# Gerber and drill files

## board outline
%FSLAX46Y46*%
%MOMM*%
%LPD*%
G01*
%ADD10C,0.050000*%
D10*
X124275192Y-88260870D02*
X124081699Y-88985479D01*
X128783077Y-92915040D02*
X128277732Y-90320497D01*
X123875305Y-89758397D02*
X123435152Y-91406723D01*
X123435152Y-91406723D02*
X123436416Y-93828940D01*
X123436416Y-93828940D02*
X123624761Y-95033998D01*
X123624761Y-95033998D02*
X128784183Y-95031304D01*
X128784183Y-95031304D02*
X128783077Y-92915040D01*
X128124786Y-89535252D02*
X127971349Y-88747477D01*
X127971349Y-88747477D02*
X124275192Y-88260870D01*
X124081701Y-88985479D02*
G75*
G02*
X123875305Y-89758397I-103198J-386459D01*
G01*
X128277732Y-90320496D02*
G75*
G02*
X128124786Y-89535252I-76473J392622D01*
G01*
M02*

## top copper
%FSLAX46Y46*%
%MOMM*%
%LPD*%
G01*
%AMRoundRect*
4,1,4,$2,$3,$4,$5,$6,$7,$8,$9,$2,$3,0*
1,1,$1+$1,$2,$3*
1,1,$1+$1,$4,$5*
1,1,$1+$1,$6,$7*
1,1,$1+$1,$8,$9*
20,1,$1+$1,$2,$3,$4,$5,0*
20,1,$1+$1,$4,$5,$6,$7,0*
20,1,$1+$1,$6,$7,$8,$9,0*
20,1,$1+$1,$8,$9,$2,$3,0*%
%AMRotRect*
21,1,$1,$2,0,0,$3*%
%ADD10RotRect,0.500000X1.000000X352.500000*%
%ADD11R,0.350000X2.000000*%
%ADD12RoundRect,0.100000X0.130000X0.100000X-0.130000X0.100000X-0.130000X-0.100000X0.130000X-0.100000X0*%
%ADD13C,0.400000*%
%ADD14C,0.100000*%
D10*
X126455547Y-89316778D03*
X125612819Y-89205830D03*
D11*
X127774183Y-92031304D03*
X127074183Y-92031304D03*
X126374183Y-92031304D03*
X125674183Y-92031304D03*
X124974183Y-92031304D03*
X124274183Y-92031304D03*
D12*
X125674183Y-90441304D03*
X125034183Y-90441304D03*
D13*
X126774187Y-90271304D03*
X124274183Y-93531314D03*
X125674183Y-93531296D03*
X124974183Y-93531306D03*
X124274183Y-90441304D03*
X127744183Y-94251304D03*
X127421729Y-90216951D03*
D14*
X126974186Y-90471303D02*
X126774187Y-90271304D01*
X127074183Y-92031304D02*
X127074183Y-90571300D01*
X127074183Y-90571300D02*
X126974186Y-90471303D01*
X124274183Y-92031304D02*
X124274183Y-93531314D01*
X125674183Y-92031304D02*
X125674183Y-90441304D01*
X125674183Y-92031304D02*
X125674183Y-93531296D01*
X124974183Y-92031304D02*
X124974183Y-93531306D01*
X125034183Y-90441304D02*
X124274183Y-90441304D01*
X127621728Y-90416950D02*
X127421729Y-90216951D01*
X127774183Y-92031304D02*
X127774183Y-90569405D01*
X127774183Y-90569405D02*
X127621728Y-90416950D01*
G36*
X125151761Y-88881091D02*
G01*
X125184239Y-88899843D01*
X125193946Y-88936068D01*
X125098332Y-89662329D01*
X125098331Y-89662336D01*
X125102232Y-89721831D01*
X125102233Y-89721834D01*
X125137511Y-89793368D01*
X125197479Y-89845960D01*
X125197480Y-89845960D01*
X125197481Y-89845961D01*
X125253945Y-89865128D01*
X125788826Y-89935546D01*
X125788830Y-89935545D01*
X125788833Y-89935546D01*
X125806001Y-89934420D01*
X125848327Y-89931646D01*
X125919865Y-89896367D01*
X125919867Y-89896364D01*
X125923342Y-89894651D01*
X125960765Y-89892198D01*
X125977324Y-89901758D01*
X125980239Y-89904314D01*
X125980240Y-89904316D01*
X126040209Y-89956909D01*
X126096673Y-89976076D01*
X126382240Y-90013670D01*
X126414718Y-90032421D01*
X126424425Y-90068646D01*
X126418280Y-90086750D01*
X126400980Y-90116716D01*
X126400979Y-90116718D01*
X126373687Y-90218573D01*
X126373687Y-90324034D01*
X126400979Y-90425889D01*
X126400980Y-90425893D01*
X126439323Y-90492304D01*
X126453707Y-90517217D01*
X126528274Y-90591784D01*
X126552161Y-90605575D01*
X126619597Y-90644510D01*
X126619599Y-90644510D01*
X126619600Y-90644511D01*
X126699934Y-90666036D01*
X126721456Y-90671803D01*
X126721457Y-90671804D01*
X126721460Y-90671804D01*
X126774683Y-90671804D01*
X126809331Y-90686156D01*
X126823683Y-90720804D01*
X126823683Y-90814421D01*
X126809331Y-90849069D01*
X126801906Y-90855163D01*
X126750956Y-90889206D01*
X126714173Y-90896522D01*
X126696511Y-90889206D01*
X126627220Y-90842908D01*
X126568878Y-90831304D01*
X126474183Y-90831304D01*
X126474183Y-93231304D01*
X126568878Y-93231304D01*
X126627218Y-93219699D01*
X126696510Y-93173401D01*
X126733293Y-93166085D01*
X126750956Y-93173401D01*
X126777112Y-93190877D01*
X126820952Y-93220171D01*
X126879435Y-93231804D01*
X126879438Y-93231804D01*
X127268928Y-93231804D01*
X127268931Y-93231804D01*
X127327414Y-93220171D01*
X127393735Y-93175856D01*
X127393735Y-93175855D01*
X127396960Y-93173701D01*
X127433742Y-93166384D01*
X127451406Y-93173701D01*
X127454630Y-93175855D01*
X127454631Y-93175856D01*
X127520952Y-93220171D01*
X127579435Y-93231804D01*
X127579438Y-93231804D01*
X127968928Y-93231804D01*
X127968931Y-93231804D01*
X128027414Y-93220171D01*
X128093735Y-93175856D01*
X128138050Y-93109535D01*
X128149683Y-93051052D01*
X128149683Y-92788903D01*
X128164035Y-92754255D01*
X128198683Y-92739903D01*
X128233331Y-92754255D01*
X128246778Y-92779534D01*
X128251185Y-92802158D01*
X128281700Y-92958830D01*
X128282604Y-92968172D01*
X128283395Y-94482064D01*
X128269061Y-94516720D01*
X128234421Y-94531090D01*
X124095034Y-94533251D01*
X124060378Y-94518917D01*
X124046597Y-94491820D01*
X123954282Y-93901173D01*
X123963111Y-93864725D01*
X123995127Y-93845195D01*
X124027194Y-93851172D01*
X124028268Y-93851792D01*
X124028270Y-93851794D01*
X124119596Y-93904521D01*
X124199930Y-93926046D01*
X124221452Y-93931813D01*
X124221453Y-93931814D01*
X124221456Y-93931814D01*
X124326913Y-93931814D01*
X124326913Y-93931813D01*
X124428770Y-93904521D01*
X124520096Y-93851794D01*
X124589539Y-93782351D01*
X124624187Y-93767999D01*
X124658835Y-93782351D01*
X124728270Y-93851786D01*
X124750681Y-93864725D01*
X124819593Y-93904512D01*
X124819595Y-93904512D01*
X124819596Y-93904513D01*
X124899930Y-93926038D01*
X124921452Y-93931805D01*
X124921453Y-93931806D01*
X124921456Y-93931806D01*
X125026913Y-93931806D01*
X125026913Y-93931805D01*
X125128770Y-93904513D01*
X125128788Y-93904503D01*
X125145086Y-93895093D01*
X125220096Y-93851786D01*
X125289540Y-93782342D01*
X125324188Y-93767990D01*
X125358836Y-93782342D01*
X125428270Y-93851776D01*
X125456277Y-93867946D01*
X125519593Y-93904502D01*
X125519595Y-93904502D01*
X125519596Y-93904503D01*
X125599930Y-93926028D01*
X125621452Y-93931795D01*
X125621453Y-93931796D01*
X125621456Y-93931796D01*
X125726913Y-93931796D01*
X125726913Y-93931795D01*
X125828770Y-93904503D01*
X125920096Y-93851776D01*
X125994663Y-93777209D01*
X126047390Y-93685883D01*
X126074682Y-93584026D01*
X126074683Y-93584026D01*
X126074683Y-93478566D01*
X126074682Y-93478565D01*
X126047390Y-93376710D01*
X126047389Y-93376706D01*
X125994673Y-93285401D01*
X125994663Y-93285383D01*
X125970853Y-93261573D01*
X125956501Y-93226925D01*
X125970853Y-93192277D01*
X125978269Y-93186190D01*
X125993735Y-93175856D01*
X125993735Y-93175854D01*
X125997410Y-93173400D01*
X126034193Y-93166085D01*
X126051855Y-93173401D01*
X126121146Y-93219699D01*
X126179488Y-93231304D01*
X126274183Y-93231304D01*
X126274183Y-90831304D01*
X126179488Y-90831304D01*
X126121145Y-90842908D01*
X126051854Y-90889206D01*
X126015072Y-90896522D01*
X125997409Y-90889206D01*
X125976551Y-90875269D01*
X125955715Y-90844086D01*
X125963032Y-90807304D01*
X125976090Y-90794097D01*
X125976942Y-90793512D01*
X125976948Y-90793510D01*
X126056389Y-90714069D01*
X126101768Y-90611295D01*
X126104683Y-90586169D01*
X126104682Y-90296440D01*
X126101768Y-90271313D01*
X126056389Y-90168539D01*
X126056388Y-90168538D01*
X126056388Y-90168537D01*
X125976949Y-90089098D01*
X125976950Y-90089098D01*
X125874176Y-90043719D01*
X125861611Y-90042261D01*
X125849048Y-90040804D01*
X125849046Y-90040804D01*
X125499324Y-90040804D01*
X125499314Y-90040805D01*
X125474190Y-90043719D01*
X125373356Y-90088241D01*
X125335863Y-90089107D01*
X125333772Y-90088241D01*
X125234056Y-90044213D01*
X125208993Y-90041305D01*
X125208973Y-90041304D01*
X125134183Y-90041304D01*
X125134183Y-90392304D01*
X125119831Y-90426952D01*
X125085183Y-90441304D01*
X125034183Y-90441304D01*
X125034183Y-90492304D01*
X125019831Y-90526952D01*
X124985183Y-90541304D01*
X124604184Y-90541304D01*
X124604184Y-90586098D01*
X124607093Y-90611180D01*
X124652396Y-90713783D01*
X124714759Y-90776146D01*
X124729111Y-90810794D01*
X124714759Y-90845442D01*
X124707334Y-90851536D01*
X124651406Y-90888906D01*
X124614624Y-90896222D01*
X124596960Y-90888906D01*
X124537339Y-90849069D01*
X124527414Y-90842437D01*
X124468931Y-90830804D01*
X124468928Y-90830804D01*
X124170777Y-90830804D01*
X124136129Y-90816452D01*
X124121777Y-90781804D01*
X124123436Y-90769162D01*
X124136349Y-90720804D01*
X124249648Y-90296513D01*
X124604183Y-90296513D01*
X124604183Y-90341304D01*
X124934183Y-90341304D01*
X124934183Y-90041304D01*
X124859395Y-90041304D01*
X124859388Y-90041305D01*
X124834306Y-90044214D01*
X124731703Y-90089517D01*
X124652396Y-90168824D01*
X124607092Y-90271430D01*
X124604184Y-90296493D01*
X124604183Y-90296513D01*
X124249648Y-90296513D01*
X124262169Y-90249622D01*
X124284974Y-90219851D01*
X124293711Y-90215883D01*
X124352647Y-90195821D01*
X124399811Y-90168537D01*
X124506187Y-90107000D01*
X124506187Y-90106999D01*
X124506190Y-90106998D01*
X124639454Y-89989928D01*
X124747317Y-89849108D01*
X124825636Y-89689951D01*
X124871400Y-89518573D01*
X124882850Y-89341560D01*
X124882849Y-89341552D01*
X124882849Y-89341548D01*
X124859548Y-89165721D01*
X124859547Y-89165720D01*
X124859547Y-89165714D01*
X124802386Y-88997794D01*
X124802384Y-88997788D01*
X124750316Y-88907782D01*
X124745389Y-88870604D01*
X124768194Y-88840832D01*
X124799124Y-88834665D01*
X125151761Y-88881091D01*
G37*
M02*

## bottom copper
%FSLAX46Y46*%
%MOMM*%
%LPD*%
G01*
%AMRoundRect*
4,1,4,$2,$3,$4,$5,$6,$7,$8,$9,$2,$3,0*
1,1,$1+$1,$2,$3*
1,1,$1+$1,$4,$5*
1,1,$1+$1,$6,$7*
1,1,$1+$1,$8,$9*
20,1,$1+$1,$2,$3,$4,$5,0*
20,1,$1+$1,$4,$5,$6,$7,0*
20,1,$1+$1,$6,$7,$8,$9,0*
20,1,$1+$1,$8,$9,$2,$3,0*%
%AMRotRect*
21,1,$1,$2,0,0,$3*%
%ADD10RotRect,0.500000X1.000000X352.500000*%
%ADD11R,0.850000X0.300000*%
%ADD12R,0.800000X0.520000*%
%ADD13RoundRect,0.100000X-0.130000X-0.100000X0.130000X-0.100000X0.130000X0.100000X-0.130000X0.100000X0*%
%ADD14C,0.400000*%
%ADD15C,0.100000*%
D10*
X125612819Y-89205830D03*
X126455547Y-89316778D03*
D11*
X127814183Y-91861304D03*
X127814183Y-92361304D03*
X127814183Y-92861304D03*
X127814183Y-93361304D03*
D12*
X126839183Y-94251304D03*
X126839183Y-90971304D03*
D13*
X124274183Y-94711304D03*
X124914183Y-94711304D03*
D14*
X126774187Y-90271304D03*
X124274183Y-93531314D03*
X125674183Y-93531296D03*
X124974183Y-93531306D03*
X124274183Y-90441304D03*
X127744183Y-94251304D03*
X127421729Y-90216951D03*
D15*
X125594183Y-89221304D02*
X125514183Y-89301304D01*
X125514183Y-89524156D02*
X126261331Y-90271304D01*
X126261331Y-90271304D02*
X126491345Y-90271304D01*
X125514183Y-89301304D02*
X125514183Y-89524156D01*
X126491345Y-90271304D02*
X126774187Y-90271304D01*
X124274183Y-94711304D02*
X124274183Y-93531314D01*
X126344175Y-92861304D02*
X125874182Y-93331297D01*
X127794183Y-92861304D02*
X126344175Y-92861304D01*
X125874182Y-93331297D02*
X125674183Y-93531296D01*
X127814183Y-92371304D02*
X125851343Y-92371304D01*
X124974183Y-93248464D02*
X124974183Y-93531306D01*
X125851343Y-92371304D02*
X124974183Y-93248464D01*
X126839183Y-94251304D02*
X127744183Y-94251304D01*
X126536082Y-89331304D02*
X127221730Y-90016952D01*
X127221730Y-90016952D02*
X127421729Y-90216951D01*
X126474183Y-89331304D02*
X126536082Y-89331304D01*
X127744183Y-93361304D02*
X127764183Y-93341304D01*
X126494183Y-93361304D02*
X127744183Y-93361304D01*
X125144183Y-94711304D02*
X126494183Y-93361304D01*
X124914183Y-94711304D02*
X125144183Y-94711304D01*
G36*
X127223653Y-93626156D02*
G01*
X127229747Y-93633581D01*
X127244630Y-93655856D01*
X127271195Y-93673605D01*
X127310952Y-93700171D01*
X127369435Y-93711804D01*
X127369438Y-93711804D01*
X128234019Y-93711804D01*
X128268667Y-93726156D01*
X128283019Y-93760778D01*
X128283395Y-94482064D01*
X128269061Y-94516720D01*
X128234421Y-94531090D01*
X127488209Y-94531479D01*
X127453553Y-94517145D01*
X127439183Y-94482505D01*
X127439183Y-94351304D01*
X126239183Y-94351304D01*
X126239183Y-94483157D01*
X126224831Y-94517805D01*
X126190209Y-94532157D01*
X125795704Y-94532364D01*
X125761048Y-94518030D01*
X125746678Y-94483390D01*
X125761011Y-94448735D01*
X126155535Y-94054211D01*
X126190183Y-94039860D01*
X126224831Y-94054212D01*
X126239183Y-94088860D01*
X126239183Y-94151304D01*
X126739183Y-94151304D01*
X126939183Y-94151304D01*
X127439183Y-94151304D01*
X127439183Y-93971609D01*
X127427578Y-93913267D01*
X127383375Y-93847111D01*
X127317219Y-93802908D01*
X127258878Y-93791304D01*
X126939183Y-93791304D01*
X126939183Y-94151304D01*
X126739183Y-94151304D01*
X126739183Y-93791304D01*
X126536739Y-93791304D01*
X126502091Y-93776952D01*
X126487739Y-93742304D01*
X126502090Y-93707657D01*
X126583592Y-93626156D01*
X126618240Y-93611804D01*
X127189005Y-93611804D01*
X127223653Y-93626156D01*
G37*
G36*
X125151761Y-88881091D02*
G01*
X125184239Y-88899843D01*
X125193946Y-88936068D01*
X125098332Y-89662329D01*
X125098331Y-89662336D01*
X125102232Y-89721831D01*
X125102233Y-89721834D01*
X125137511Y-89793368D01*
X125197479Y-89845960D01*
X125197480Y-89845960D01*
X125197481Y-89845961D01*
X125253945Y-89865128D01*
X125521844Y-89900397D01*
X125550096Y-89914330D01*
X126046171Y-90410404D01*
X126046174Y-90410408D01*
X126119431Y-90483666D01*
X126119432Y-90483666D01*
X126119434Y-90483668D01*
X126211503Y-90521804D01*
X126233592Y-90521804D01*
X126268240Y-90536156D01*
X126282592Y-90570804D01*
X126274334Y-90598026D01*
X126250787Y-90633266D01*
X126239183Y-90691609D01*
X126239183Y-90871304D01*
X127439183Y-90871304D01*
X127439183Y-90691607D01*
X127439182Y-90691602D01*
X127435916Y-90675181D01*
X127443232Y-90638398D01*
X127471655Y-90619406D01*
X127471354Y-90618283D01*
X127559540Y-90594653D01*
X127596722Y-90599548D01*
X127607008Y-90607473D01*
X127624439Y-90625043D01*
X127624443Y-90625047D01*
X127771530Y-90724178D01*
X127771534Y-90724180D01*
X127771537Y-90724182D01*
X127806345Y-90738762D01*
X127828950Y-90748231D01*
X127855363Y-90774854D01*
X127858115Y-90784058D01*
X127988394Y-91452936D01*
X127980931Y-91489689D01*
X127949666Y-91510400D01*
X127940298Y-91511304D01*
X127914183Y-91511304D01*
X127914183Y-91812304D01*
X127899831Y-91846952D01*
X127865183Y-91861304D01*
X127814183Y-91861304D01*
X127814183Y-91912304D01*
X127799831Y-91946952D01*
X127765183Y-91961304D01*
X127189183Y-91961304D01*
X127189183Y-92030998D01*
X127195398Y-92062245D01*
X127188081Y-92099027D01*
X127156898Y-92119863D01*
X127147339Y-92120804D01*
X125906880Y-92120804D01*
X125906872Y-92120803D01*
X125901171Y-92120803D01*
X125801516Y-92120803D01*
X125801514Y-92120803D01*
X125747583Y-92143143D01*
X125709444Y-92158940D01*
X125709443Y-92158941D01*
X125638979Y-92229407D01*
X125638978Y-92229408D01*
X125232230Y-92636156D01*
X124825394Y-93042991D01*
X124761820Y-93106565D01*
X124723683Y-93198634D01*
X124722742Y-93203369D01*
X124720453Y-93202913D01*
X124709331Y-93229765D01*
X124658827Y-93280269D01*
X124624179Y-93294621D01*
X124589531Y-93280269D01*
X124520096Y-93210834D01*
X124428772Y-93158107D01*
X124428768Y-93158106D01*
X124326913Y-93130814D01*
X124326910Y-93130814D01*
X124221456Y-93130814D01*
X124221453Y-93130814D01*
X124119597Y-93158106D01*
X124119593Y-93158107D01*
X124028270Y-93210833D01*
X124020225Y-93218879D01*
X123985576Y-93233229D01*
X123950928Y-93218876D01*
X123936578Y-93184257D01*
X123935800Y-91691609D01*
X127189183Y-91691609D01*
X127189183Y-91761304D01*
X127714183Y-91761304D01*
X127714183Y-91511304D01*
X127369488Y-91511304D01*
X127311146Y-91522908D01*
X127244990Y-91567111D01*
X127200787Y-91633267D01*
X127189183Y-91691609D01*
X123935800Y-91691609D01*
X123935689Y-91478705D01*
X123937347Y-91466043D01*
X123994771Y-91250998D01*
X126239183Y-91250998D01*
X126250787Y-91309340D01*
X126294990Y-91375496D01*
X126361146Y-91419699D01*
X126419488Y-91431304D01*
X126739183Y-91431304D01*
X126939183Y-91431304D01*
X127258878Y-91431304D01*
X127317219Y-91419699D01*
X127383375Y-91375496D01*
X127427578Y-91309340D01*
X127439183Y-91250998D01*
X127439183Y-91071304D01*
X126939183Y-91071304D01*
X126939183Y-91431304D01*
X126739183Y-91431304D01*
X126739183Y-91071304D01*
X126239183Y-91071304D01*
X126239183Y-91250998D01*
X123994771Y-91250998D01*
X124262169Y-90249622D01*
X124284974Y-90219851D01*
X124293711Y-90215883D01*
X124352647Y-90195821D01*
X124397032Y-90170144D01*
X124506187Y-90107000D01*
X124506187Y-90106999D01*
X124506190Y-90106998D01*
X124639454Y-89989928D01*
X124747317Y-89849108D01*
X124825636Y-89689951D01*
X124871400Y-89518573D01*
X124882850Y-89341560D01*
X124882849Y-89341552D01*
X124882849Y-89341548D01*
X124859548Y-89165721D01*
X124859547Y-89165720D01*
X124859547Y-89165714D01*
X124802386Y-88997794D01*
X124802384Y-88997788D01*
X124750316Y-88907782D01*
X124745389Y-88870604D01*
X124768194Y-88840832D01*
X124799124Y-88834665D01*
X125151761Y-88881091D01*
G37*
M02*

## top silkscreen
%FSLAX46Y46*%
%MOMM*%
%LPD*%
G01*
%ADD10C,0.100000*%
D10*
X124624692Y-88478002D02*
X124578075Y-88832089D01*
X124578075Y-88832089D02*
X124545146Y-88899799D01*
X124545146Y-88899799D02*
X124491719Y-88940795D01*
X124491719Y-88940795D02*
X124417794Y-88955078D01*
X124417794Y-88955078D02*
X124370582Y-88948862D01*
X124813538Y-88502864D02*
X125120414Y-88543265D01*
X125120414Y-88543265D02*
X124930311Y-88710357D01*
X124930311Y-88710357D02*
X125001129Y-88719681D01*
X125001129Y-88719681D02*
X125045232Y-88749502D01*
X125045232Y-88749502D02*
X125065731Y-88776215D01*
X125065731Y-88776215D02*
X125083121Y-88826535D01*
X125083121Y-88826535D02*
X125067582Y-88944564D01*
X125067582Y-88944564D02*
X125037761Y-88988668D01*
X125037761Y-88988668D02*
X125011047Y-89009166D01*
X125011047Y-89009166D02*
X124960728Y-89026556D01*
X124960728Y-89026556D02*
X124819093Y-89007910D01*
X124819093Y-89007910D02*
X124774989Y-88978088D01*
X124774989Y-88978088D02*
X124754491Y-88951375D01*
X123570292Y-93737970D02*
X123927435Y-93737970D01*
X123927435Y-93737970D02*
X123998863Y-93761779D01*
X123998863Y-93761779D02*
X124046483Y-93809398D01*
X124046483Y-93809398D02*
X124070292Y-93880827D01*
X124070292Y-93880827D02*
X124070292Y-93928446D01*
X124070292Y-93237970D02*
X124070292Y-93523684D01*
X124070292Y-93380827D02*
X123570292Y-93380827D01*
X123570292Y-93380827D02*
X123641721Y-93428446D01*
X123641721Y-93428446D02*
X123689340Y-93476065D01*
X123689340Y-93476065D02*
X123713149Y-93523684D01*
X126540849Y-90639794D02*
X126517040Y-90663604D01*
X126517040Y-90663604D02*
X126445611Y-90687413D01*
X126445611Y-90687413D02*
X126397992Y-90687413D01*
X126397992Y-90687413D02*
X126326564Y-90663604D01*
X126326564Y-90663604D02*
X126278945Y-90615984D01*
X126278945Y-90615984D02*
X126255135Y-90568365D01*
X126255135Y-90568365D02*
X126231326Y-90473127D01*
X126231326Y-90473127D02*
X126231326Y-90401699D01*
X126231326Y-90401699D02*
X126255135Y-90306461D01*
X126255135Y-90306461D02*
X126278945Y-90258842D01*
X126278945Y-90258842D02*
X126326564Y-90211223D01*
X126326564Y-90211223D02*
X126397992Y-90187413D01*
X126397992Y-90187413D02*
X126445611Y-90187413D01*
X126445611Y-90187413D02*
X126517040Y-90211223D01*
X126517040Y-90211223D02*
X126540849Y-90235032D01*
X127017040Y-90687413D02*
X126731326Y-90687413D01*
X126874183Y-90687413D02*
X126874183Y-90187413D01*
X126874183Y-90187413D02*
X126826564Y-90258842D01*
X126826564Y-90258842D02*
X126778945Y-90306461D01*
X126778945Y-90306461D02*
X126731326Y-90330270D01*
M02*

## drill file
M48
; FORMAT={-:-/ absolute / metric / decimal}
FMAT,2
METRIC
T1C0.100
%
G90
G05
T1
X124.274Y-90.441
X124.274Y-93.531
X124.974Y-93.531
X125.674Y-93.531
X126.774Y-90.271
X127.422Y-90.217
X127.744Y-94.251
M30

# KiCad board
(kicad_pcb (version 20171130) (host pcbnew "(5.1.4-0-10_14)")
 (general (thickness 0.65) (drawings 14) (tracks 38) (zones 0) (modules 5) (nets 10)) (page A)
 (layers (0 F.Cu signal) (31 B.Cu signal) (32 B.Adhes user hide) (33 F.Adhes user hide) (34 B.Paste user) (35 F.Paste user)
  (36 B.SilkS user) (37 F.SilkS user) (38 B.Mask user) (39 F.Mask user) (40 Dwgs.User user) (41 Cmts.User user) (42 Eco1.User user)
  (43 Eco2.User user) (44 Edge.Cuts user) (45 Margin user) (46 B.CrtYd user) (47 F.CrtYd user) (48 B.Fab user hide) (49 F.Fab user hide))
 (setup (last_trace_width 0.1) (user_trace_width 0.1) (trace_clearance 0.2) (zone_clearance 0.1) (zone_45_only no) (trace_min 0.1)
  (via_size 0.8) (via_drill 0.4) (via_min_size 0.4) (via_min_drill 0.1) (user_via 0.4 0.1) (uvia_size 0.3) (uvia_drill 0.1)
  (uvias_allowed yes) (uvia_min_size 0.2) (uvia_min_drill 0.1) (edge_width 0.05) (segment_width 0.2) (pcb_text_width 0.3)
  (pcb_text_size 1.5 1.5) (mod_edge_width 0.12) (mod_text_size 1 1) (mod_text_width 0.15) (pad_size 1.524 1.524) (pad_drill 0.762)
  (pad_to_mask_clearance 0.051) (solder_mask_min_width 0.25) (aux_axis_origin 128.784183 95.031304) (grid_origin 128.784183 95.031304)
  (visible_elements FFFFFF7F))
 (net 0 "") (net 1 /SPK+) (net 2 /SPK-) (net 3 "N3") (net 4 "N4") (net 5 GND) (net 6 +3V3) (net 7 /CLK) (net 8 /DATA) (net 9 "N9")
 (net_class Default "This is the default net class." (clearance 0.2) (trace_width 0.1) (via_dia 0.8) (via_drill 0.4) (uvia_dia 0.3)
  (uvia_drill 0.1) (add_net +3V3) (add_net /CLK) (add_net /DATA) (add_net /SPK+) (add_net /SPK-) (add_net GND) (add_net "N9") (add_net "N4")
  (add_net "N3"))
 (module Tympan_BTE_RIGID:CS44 (layer F.Cu) (at 126.034183 89.261304 352.5)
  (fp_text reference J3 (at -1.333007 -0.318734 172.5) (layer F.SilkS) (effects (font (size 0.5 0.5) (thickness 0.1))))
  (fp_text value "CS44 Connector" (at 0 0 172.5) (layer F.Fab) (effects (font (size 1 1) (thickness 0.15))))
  (pad 4 smd rect (at -0.425 0 352.5) (size 0.5 1) (layers B.Cu B.Mask) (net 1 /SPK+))
  (pad 3 smd rect (at 0.425 0 352.5) (size 0.5 1) (layers B.Cu B.Mask) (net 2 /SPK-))
  (pad 2 smd rect (at 0.425 0 352.5) (size 0.5 1) (layers F.Cu F.Mask) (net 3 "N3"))
  (pad 1 smd rect (at -0.425 0 352.5) (size 0.5 1) (layers F.Cu F.Mask) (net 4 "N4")))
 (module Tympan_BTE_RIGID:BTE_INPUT (layer F.Cu) (at 126.024183 92.031304 90)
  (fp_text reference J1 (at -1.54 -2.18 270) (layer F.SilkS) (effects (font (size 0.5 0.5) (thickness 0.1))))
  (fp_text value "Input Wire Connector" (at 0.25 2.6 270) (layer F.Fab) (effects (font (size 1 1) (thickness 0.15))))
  (pad 6 smd rect (at 0 1.75 90) (size 2 0.35) (layers F.Cu F.Mask) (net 2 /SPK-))
  (pad 5 smd rect (at 0 1.05 90) (size 2 0.35) (layers F.Cu F.Mask) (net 1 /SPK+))
  (pad 4 smd rect (at 0 0.35 90) (size 2 0.35) (layers F.Cu F.Mask) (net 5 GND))
  (pad 3 smd rect (at 0 -0.35 90) (size 2 0.35) (layers F.Cu F.Mask) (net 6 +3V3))
  (pad 2 smd rect (at 0 -1.05 90) (size 2 0.35) (layers F.Cu F.Mask) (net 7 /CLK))
  (pad 1 smd rect (at 0 -1.75 90) (size 2 0.35) (layers F.Cu F.Mask) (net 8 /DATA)))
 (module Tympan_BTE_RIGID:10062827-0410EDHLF (layer B.Cu) (at 127.814183 92.611304 90)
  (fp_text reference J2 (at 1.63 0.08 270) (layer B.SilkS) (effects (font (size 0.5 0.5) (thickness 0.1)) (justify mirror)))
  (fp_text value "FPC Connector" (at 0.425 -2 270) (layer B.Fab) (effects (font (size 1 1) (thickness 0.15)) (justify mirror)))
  (pad 1 smd rect (at 0.75 0 90) (size 0.3 0.85) (layers B.Cu B.Paste B.Mask) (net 5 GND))
  (pad 2 smd rect (at 0.25 0 90) (size 0.3 0.85) (layers B.Cu B.Paste B.Mask) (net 7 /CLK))
  (pad 3 smd rect (at -0.25 0 90) (size 0.3 0.85) (layers B.Cu B.Paste B.Mask) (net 6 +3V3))
  (pad 4 smd rect (at -0.75 0 90) (size 0.3 0.85) (layers B.Cu B.Paste B.Mask) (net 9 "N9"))
  (pad 5 smd rect (at -1.64 -0.975 90) (size 0.52 0.8) (layers B.Cu B.Paste B.Mask) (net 5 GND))
  (pad 6 smd rect (at 1.64 -0.975 90) (size 0.52 0.8) (layers B.Cu B.Paste B.Mask) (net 5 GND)))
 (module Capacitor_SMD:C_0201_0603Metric (layer F.Cu) (at 125.354183 90.441304 180)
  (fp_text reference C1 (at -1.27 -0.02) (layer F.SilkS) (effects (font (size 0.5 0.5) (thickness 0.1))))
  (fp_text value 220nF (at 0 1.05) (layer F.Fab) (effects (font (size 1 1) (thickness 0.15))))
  (pad "" smd roundrect (at -0.345 0 180) (size 0.318 0.36) (layers F.Paste) (roundrect_rratio 0.25))
  (pad "" smd roundrect (at 0.345 0 180) (size 0.318 0.36) (layers F.Paste) (roundrect_rratio 0.25))
  (pad 1 smd roundrect (at -0.32 0 180) (size 0.46 0.4) (layers F.Cu F.Mask) (roundrect_rratio 0.25) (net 6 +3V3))
  (pad 2 smd roundrect (at 0.32 0 180) (size 0.46 0.4) (layers F.Cu F.Mask) (roundrect_rratio 0.25) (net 5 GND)))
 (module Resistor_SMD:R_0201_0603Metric (layer B.Cu) (at 124.594183 94.711304)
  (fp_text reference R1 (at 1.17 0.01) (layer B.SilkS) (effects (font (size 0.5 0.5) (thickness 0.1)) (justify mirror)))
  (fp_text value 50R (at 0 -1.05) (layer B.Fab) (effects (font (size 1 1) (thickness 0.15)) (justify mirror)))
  (pad "" smd roundrect (at -0.345 0) (size 0.318 0.36) (layers B.Paste) (roundrect_rratio 0.25))
  (pad "" smd roundrect (at 0.345 0) (size 0.318 0.36) (layers B.Paste) (roundrect_rratio 0.25))
  (pad 1 smd roundrect (at -0.32 0) (size 0.46 0.4) (layers B.Cu B.Mask) (roundrect_rratio 0.25) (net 8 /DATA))
  (pad 2 smd roundrect (at 0.32 0) (size 0.46 0.4) (layers B.Cu B.Mask) (roundrect_rratio 0.25) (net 9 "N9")))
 (gr_line (start 124.275192 88.26087) (end 124.081699 88.985479) (layer Edge.Cuts) (width 0.05))
 (gr_line (start 128.783077 92.91504) (end 128.277732 90.320497) (layer Edge.Cuts) (width 0.05))
 (gr_line (start 123.875305 89.758397) (end 123.435152 91.406723) (layer Edge.Cuts) (width 0.05))
 (gr_line (start 123.435152 91.406723) (end 123.436416 93.82894) (layer Edge.Cuts) (width 0.05))
 (gr_line (start 123.436416 93.82894) (end 123.624761 95.033998) (layer Edge.Cuts) (width 0.05))
 (gr_line (start 123.624761 95.033998) (end 128.784183 95.031304) (layer Edge.Cuts) (width 0.05))
 (gr_line (start 128.784183 95.031304) (end 128.783077 92.91504) (layer Edge.Cuts) (width 0.05))
 (gr_line (start 128.124786 89.535252) (end 127.971349 88.747477) (layer Edge.Cuts) (width 0.05))
 (gr_line (start 127.971349 88.747477) (end 124.275192 88.26087) (layer Edge.Cuts) (width 0.05))
 (gr_arc (start 123.978503 89.371938) (end 123.875305 89.758397) (angle -180) (layer Edge.Cuts) (width 0.05))
 (gr_arc (start 128.201259 89.927874) (end 128.124786 89.535252) (angle -180) (layer Edge.Cuts) (width 0.05))
 (via (at 126.774187 90.271304) (size 0.4) (drill 0.1) (layers F.Cu B.Cu) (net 1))
 (segment (start 126.974186 90.471303) (end 126.774187 90.271304) (width 0.1) (layer F.Cu) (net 1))
 (segment (start 125.594183 89.221304) (end 125.514183 89.301304) (width 0.1) (layer B.Cu) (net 1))
 (segment (start 127.074183 92.031304) (end 127.074183 90.5713) (width 0.1) (layer F.Cu) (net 1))
 (segment (start 127.074183 90.5713) (end 126.974186 90.471303) (width 0.1) (layer F.Cu) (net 1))
 (segment (start 125.514183 89.524156) (end 126.261331 90.271304) (width 0.1) (layer B.Cu) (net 1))
 (segment (start 126.261331 90.271304) (end 126.491345 90.271304) (width 0.1) (layer B.Cu) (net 1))
 (segment (start 125.514183 89.301304) (end 125.514183 89.524156) (width 0.1) (layer B.Cu) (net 1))
 (segment (start 126.491345 90.271304) (end 126.774187 90.271304) (width 0.1) (layer B.Cu) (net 1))
 (via (at 124.274183 93.531314) (size 0.4) (drill 0.1) (layers F.Cu B.Cu) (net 8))
 (segment (start 124.274183 92.031304) (end 124.274183 93.531314) (width 0.1) (layer F.Cu) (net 8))
 (segment (start 124.274183 94.711304) (end 124.274183 93.531314) (width 0.1) (layer B.Cu) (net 8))
 (segment (start 125.674183 92.031304) (end 125.674183 90.441304) (width 0.1) (layer F.Cu) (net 6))
 (via (at 125.674183 93.531296) (size 0.4) (drill 0.1) (layers F.Cu B.Cu) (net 6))
 (segment (start 126.344175 92.861304) (end 125.874182 93.331297) (width 0.1) (layer B.Cu) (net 6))
 (segment (start 125.674183 92.031304) (end 125.674183 93.531296) (width 0.1) (layer F.Cu) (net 6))
 (segment (start 127.794183 92.861304) (end 126.344175 92.861304) (width 0.1) (layer B.Cu) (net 6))
 (segment (start 125.874182 93.331297) (end 125.674183 93.531296) (width 0.1) (layer B.Cu) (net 6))
 (via (at 124.974183 93.531306) (size 0.4) (drill 0.1) (layers F.Cu B.Cu) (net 7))
 (segment (start 124.974183 92.031304) (end 124.974183 93.531306) (width 0.1) (layer F.Cu) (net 7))
 (segment (start 127.814183 92.371304) (end 125.851343 92.371304) (width 0.1) (layer B.Cu) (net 7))
 (segment (start 124.974183 93.248464) (end 124.974183 93.531306) (width 0.1) (layer B.Cu) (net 7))
 (segment (start 125.851343 92.371304) (end 124.974183 93.248464) (width 0.1) (layer B.Cu) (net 7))
 (via (at 124.274183 90.441304) (size 0.4) (drill 0.1) (layers F.Cu B.Cu) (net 5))
 (segment (start 125.034183 90.441304) (end 124.274183 90.441304) (width 0.1) (layer F.Cu) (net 5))
 (via (at 127.744183 94.251304) (size 0.4) (drill 0.1) (layers F.Cu B.Cu) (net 5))
 (segment (start 126.839183 94.251304) (end 127.744183 94.251304) (width 0.1) (layer B.Cu) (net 5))
 (segment (start 126.536082 89.331304) (end 127.22173 90.016952) (width 0.1) (layer B.Cu) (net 2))
 (segment (start 127.621728 90.41695) (end 127.421729 90.216951) (width 0.1) (layer F.Cu) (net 2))
 (via (at 127.421729 90.216951) (size 0.4) (drill 0.1) (layers F.Cu B.Cu) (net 2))
 (segment (start 127.22173 90.016952) (end 127.421729 90.216951) (width 0.1) (layer B.Cu) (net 2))
 (segment (start 127.774183 92.031304) (end 127.774183 90.569405) (width 0.1) (layer F.Cu) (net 2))
 (segment (start 127.774183 90.569405) (end 127.621728 90.41695) (width 0.1) (layer F.Cu) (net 2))
 (segment (start 126.474183 89.331304) (end 126.536082 89.331304) (width 0.1) (layer B.Cu) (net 2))
 (segment (start 127.744183 93.361304) (end 127.764183 93.341304) (width 0.1) (layer B.Cu) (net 9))
 (segment (start 126.494183 93.361304) (end 127.744183 93.361304) (width 0.1) (layer B.Cu) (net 9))
 (segment (start 125.144183 94.711304) (end 126.494183 93.361304) (width 0.1) (layer B.Cu) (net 9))
 (segment (start 124.914183 94.711304) (end 125.144183 94.711304) (width 0.1) (layer B.Cu) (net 9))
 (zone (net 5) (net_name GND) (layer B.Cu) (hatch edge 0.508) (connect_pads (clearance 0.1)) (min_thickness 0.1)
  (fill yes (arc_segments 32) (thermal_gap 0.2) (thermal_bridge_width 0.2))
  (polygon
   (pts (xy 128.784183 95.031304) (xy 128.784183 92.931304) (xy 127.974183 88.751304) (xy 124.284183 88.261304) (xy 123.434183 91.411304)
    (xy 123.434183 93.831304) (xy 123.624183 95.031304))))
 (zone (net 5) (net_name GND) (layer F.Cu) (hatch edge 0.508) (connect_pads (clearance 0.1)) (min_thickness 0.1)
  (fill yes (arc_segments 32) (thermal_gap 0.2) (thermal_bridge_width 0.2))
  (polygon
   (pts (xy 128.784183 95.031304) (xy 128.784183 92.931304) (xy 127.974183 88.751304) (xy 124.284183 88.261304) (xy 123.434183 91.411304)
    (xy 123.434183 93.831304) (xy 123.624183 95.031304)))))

